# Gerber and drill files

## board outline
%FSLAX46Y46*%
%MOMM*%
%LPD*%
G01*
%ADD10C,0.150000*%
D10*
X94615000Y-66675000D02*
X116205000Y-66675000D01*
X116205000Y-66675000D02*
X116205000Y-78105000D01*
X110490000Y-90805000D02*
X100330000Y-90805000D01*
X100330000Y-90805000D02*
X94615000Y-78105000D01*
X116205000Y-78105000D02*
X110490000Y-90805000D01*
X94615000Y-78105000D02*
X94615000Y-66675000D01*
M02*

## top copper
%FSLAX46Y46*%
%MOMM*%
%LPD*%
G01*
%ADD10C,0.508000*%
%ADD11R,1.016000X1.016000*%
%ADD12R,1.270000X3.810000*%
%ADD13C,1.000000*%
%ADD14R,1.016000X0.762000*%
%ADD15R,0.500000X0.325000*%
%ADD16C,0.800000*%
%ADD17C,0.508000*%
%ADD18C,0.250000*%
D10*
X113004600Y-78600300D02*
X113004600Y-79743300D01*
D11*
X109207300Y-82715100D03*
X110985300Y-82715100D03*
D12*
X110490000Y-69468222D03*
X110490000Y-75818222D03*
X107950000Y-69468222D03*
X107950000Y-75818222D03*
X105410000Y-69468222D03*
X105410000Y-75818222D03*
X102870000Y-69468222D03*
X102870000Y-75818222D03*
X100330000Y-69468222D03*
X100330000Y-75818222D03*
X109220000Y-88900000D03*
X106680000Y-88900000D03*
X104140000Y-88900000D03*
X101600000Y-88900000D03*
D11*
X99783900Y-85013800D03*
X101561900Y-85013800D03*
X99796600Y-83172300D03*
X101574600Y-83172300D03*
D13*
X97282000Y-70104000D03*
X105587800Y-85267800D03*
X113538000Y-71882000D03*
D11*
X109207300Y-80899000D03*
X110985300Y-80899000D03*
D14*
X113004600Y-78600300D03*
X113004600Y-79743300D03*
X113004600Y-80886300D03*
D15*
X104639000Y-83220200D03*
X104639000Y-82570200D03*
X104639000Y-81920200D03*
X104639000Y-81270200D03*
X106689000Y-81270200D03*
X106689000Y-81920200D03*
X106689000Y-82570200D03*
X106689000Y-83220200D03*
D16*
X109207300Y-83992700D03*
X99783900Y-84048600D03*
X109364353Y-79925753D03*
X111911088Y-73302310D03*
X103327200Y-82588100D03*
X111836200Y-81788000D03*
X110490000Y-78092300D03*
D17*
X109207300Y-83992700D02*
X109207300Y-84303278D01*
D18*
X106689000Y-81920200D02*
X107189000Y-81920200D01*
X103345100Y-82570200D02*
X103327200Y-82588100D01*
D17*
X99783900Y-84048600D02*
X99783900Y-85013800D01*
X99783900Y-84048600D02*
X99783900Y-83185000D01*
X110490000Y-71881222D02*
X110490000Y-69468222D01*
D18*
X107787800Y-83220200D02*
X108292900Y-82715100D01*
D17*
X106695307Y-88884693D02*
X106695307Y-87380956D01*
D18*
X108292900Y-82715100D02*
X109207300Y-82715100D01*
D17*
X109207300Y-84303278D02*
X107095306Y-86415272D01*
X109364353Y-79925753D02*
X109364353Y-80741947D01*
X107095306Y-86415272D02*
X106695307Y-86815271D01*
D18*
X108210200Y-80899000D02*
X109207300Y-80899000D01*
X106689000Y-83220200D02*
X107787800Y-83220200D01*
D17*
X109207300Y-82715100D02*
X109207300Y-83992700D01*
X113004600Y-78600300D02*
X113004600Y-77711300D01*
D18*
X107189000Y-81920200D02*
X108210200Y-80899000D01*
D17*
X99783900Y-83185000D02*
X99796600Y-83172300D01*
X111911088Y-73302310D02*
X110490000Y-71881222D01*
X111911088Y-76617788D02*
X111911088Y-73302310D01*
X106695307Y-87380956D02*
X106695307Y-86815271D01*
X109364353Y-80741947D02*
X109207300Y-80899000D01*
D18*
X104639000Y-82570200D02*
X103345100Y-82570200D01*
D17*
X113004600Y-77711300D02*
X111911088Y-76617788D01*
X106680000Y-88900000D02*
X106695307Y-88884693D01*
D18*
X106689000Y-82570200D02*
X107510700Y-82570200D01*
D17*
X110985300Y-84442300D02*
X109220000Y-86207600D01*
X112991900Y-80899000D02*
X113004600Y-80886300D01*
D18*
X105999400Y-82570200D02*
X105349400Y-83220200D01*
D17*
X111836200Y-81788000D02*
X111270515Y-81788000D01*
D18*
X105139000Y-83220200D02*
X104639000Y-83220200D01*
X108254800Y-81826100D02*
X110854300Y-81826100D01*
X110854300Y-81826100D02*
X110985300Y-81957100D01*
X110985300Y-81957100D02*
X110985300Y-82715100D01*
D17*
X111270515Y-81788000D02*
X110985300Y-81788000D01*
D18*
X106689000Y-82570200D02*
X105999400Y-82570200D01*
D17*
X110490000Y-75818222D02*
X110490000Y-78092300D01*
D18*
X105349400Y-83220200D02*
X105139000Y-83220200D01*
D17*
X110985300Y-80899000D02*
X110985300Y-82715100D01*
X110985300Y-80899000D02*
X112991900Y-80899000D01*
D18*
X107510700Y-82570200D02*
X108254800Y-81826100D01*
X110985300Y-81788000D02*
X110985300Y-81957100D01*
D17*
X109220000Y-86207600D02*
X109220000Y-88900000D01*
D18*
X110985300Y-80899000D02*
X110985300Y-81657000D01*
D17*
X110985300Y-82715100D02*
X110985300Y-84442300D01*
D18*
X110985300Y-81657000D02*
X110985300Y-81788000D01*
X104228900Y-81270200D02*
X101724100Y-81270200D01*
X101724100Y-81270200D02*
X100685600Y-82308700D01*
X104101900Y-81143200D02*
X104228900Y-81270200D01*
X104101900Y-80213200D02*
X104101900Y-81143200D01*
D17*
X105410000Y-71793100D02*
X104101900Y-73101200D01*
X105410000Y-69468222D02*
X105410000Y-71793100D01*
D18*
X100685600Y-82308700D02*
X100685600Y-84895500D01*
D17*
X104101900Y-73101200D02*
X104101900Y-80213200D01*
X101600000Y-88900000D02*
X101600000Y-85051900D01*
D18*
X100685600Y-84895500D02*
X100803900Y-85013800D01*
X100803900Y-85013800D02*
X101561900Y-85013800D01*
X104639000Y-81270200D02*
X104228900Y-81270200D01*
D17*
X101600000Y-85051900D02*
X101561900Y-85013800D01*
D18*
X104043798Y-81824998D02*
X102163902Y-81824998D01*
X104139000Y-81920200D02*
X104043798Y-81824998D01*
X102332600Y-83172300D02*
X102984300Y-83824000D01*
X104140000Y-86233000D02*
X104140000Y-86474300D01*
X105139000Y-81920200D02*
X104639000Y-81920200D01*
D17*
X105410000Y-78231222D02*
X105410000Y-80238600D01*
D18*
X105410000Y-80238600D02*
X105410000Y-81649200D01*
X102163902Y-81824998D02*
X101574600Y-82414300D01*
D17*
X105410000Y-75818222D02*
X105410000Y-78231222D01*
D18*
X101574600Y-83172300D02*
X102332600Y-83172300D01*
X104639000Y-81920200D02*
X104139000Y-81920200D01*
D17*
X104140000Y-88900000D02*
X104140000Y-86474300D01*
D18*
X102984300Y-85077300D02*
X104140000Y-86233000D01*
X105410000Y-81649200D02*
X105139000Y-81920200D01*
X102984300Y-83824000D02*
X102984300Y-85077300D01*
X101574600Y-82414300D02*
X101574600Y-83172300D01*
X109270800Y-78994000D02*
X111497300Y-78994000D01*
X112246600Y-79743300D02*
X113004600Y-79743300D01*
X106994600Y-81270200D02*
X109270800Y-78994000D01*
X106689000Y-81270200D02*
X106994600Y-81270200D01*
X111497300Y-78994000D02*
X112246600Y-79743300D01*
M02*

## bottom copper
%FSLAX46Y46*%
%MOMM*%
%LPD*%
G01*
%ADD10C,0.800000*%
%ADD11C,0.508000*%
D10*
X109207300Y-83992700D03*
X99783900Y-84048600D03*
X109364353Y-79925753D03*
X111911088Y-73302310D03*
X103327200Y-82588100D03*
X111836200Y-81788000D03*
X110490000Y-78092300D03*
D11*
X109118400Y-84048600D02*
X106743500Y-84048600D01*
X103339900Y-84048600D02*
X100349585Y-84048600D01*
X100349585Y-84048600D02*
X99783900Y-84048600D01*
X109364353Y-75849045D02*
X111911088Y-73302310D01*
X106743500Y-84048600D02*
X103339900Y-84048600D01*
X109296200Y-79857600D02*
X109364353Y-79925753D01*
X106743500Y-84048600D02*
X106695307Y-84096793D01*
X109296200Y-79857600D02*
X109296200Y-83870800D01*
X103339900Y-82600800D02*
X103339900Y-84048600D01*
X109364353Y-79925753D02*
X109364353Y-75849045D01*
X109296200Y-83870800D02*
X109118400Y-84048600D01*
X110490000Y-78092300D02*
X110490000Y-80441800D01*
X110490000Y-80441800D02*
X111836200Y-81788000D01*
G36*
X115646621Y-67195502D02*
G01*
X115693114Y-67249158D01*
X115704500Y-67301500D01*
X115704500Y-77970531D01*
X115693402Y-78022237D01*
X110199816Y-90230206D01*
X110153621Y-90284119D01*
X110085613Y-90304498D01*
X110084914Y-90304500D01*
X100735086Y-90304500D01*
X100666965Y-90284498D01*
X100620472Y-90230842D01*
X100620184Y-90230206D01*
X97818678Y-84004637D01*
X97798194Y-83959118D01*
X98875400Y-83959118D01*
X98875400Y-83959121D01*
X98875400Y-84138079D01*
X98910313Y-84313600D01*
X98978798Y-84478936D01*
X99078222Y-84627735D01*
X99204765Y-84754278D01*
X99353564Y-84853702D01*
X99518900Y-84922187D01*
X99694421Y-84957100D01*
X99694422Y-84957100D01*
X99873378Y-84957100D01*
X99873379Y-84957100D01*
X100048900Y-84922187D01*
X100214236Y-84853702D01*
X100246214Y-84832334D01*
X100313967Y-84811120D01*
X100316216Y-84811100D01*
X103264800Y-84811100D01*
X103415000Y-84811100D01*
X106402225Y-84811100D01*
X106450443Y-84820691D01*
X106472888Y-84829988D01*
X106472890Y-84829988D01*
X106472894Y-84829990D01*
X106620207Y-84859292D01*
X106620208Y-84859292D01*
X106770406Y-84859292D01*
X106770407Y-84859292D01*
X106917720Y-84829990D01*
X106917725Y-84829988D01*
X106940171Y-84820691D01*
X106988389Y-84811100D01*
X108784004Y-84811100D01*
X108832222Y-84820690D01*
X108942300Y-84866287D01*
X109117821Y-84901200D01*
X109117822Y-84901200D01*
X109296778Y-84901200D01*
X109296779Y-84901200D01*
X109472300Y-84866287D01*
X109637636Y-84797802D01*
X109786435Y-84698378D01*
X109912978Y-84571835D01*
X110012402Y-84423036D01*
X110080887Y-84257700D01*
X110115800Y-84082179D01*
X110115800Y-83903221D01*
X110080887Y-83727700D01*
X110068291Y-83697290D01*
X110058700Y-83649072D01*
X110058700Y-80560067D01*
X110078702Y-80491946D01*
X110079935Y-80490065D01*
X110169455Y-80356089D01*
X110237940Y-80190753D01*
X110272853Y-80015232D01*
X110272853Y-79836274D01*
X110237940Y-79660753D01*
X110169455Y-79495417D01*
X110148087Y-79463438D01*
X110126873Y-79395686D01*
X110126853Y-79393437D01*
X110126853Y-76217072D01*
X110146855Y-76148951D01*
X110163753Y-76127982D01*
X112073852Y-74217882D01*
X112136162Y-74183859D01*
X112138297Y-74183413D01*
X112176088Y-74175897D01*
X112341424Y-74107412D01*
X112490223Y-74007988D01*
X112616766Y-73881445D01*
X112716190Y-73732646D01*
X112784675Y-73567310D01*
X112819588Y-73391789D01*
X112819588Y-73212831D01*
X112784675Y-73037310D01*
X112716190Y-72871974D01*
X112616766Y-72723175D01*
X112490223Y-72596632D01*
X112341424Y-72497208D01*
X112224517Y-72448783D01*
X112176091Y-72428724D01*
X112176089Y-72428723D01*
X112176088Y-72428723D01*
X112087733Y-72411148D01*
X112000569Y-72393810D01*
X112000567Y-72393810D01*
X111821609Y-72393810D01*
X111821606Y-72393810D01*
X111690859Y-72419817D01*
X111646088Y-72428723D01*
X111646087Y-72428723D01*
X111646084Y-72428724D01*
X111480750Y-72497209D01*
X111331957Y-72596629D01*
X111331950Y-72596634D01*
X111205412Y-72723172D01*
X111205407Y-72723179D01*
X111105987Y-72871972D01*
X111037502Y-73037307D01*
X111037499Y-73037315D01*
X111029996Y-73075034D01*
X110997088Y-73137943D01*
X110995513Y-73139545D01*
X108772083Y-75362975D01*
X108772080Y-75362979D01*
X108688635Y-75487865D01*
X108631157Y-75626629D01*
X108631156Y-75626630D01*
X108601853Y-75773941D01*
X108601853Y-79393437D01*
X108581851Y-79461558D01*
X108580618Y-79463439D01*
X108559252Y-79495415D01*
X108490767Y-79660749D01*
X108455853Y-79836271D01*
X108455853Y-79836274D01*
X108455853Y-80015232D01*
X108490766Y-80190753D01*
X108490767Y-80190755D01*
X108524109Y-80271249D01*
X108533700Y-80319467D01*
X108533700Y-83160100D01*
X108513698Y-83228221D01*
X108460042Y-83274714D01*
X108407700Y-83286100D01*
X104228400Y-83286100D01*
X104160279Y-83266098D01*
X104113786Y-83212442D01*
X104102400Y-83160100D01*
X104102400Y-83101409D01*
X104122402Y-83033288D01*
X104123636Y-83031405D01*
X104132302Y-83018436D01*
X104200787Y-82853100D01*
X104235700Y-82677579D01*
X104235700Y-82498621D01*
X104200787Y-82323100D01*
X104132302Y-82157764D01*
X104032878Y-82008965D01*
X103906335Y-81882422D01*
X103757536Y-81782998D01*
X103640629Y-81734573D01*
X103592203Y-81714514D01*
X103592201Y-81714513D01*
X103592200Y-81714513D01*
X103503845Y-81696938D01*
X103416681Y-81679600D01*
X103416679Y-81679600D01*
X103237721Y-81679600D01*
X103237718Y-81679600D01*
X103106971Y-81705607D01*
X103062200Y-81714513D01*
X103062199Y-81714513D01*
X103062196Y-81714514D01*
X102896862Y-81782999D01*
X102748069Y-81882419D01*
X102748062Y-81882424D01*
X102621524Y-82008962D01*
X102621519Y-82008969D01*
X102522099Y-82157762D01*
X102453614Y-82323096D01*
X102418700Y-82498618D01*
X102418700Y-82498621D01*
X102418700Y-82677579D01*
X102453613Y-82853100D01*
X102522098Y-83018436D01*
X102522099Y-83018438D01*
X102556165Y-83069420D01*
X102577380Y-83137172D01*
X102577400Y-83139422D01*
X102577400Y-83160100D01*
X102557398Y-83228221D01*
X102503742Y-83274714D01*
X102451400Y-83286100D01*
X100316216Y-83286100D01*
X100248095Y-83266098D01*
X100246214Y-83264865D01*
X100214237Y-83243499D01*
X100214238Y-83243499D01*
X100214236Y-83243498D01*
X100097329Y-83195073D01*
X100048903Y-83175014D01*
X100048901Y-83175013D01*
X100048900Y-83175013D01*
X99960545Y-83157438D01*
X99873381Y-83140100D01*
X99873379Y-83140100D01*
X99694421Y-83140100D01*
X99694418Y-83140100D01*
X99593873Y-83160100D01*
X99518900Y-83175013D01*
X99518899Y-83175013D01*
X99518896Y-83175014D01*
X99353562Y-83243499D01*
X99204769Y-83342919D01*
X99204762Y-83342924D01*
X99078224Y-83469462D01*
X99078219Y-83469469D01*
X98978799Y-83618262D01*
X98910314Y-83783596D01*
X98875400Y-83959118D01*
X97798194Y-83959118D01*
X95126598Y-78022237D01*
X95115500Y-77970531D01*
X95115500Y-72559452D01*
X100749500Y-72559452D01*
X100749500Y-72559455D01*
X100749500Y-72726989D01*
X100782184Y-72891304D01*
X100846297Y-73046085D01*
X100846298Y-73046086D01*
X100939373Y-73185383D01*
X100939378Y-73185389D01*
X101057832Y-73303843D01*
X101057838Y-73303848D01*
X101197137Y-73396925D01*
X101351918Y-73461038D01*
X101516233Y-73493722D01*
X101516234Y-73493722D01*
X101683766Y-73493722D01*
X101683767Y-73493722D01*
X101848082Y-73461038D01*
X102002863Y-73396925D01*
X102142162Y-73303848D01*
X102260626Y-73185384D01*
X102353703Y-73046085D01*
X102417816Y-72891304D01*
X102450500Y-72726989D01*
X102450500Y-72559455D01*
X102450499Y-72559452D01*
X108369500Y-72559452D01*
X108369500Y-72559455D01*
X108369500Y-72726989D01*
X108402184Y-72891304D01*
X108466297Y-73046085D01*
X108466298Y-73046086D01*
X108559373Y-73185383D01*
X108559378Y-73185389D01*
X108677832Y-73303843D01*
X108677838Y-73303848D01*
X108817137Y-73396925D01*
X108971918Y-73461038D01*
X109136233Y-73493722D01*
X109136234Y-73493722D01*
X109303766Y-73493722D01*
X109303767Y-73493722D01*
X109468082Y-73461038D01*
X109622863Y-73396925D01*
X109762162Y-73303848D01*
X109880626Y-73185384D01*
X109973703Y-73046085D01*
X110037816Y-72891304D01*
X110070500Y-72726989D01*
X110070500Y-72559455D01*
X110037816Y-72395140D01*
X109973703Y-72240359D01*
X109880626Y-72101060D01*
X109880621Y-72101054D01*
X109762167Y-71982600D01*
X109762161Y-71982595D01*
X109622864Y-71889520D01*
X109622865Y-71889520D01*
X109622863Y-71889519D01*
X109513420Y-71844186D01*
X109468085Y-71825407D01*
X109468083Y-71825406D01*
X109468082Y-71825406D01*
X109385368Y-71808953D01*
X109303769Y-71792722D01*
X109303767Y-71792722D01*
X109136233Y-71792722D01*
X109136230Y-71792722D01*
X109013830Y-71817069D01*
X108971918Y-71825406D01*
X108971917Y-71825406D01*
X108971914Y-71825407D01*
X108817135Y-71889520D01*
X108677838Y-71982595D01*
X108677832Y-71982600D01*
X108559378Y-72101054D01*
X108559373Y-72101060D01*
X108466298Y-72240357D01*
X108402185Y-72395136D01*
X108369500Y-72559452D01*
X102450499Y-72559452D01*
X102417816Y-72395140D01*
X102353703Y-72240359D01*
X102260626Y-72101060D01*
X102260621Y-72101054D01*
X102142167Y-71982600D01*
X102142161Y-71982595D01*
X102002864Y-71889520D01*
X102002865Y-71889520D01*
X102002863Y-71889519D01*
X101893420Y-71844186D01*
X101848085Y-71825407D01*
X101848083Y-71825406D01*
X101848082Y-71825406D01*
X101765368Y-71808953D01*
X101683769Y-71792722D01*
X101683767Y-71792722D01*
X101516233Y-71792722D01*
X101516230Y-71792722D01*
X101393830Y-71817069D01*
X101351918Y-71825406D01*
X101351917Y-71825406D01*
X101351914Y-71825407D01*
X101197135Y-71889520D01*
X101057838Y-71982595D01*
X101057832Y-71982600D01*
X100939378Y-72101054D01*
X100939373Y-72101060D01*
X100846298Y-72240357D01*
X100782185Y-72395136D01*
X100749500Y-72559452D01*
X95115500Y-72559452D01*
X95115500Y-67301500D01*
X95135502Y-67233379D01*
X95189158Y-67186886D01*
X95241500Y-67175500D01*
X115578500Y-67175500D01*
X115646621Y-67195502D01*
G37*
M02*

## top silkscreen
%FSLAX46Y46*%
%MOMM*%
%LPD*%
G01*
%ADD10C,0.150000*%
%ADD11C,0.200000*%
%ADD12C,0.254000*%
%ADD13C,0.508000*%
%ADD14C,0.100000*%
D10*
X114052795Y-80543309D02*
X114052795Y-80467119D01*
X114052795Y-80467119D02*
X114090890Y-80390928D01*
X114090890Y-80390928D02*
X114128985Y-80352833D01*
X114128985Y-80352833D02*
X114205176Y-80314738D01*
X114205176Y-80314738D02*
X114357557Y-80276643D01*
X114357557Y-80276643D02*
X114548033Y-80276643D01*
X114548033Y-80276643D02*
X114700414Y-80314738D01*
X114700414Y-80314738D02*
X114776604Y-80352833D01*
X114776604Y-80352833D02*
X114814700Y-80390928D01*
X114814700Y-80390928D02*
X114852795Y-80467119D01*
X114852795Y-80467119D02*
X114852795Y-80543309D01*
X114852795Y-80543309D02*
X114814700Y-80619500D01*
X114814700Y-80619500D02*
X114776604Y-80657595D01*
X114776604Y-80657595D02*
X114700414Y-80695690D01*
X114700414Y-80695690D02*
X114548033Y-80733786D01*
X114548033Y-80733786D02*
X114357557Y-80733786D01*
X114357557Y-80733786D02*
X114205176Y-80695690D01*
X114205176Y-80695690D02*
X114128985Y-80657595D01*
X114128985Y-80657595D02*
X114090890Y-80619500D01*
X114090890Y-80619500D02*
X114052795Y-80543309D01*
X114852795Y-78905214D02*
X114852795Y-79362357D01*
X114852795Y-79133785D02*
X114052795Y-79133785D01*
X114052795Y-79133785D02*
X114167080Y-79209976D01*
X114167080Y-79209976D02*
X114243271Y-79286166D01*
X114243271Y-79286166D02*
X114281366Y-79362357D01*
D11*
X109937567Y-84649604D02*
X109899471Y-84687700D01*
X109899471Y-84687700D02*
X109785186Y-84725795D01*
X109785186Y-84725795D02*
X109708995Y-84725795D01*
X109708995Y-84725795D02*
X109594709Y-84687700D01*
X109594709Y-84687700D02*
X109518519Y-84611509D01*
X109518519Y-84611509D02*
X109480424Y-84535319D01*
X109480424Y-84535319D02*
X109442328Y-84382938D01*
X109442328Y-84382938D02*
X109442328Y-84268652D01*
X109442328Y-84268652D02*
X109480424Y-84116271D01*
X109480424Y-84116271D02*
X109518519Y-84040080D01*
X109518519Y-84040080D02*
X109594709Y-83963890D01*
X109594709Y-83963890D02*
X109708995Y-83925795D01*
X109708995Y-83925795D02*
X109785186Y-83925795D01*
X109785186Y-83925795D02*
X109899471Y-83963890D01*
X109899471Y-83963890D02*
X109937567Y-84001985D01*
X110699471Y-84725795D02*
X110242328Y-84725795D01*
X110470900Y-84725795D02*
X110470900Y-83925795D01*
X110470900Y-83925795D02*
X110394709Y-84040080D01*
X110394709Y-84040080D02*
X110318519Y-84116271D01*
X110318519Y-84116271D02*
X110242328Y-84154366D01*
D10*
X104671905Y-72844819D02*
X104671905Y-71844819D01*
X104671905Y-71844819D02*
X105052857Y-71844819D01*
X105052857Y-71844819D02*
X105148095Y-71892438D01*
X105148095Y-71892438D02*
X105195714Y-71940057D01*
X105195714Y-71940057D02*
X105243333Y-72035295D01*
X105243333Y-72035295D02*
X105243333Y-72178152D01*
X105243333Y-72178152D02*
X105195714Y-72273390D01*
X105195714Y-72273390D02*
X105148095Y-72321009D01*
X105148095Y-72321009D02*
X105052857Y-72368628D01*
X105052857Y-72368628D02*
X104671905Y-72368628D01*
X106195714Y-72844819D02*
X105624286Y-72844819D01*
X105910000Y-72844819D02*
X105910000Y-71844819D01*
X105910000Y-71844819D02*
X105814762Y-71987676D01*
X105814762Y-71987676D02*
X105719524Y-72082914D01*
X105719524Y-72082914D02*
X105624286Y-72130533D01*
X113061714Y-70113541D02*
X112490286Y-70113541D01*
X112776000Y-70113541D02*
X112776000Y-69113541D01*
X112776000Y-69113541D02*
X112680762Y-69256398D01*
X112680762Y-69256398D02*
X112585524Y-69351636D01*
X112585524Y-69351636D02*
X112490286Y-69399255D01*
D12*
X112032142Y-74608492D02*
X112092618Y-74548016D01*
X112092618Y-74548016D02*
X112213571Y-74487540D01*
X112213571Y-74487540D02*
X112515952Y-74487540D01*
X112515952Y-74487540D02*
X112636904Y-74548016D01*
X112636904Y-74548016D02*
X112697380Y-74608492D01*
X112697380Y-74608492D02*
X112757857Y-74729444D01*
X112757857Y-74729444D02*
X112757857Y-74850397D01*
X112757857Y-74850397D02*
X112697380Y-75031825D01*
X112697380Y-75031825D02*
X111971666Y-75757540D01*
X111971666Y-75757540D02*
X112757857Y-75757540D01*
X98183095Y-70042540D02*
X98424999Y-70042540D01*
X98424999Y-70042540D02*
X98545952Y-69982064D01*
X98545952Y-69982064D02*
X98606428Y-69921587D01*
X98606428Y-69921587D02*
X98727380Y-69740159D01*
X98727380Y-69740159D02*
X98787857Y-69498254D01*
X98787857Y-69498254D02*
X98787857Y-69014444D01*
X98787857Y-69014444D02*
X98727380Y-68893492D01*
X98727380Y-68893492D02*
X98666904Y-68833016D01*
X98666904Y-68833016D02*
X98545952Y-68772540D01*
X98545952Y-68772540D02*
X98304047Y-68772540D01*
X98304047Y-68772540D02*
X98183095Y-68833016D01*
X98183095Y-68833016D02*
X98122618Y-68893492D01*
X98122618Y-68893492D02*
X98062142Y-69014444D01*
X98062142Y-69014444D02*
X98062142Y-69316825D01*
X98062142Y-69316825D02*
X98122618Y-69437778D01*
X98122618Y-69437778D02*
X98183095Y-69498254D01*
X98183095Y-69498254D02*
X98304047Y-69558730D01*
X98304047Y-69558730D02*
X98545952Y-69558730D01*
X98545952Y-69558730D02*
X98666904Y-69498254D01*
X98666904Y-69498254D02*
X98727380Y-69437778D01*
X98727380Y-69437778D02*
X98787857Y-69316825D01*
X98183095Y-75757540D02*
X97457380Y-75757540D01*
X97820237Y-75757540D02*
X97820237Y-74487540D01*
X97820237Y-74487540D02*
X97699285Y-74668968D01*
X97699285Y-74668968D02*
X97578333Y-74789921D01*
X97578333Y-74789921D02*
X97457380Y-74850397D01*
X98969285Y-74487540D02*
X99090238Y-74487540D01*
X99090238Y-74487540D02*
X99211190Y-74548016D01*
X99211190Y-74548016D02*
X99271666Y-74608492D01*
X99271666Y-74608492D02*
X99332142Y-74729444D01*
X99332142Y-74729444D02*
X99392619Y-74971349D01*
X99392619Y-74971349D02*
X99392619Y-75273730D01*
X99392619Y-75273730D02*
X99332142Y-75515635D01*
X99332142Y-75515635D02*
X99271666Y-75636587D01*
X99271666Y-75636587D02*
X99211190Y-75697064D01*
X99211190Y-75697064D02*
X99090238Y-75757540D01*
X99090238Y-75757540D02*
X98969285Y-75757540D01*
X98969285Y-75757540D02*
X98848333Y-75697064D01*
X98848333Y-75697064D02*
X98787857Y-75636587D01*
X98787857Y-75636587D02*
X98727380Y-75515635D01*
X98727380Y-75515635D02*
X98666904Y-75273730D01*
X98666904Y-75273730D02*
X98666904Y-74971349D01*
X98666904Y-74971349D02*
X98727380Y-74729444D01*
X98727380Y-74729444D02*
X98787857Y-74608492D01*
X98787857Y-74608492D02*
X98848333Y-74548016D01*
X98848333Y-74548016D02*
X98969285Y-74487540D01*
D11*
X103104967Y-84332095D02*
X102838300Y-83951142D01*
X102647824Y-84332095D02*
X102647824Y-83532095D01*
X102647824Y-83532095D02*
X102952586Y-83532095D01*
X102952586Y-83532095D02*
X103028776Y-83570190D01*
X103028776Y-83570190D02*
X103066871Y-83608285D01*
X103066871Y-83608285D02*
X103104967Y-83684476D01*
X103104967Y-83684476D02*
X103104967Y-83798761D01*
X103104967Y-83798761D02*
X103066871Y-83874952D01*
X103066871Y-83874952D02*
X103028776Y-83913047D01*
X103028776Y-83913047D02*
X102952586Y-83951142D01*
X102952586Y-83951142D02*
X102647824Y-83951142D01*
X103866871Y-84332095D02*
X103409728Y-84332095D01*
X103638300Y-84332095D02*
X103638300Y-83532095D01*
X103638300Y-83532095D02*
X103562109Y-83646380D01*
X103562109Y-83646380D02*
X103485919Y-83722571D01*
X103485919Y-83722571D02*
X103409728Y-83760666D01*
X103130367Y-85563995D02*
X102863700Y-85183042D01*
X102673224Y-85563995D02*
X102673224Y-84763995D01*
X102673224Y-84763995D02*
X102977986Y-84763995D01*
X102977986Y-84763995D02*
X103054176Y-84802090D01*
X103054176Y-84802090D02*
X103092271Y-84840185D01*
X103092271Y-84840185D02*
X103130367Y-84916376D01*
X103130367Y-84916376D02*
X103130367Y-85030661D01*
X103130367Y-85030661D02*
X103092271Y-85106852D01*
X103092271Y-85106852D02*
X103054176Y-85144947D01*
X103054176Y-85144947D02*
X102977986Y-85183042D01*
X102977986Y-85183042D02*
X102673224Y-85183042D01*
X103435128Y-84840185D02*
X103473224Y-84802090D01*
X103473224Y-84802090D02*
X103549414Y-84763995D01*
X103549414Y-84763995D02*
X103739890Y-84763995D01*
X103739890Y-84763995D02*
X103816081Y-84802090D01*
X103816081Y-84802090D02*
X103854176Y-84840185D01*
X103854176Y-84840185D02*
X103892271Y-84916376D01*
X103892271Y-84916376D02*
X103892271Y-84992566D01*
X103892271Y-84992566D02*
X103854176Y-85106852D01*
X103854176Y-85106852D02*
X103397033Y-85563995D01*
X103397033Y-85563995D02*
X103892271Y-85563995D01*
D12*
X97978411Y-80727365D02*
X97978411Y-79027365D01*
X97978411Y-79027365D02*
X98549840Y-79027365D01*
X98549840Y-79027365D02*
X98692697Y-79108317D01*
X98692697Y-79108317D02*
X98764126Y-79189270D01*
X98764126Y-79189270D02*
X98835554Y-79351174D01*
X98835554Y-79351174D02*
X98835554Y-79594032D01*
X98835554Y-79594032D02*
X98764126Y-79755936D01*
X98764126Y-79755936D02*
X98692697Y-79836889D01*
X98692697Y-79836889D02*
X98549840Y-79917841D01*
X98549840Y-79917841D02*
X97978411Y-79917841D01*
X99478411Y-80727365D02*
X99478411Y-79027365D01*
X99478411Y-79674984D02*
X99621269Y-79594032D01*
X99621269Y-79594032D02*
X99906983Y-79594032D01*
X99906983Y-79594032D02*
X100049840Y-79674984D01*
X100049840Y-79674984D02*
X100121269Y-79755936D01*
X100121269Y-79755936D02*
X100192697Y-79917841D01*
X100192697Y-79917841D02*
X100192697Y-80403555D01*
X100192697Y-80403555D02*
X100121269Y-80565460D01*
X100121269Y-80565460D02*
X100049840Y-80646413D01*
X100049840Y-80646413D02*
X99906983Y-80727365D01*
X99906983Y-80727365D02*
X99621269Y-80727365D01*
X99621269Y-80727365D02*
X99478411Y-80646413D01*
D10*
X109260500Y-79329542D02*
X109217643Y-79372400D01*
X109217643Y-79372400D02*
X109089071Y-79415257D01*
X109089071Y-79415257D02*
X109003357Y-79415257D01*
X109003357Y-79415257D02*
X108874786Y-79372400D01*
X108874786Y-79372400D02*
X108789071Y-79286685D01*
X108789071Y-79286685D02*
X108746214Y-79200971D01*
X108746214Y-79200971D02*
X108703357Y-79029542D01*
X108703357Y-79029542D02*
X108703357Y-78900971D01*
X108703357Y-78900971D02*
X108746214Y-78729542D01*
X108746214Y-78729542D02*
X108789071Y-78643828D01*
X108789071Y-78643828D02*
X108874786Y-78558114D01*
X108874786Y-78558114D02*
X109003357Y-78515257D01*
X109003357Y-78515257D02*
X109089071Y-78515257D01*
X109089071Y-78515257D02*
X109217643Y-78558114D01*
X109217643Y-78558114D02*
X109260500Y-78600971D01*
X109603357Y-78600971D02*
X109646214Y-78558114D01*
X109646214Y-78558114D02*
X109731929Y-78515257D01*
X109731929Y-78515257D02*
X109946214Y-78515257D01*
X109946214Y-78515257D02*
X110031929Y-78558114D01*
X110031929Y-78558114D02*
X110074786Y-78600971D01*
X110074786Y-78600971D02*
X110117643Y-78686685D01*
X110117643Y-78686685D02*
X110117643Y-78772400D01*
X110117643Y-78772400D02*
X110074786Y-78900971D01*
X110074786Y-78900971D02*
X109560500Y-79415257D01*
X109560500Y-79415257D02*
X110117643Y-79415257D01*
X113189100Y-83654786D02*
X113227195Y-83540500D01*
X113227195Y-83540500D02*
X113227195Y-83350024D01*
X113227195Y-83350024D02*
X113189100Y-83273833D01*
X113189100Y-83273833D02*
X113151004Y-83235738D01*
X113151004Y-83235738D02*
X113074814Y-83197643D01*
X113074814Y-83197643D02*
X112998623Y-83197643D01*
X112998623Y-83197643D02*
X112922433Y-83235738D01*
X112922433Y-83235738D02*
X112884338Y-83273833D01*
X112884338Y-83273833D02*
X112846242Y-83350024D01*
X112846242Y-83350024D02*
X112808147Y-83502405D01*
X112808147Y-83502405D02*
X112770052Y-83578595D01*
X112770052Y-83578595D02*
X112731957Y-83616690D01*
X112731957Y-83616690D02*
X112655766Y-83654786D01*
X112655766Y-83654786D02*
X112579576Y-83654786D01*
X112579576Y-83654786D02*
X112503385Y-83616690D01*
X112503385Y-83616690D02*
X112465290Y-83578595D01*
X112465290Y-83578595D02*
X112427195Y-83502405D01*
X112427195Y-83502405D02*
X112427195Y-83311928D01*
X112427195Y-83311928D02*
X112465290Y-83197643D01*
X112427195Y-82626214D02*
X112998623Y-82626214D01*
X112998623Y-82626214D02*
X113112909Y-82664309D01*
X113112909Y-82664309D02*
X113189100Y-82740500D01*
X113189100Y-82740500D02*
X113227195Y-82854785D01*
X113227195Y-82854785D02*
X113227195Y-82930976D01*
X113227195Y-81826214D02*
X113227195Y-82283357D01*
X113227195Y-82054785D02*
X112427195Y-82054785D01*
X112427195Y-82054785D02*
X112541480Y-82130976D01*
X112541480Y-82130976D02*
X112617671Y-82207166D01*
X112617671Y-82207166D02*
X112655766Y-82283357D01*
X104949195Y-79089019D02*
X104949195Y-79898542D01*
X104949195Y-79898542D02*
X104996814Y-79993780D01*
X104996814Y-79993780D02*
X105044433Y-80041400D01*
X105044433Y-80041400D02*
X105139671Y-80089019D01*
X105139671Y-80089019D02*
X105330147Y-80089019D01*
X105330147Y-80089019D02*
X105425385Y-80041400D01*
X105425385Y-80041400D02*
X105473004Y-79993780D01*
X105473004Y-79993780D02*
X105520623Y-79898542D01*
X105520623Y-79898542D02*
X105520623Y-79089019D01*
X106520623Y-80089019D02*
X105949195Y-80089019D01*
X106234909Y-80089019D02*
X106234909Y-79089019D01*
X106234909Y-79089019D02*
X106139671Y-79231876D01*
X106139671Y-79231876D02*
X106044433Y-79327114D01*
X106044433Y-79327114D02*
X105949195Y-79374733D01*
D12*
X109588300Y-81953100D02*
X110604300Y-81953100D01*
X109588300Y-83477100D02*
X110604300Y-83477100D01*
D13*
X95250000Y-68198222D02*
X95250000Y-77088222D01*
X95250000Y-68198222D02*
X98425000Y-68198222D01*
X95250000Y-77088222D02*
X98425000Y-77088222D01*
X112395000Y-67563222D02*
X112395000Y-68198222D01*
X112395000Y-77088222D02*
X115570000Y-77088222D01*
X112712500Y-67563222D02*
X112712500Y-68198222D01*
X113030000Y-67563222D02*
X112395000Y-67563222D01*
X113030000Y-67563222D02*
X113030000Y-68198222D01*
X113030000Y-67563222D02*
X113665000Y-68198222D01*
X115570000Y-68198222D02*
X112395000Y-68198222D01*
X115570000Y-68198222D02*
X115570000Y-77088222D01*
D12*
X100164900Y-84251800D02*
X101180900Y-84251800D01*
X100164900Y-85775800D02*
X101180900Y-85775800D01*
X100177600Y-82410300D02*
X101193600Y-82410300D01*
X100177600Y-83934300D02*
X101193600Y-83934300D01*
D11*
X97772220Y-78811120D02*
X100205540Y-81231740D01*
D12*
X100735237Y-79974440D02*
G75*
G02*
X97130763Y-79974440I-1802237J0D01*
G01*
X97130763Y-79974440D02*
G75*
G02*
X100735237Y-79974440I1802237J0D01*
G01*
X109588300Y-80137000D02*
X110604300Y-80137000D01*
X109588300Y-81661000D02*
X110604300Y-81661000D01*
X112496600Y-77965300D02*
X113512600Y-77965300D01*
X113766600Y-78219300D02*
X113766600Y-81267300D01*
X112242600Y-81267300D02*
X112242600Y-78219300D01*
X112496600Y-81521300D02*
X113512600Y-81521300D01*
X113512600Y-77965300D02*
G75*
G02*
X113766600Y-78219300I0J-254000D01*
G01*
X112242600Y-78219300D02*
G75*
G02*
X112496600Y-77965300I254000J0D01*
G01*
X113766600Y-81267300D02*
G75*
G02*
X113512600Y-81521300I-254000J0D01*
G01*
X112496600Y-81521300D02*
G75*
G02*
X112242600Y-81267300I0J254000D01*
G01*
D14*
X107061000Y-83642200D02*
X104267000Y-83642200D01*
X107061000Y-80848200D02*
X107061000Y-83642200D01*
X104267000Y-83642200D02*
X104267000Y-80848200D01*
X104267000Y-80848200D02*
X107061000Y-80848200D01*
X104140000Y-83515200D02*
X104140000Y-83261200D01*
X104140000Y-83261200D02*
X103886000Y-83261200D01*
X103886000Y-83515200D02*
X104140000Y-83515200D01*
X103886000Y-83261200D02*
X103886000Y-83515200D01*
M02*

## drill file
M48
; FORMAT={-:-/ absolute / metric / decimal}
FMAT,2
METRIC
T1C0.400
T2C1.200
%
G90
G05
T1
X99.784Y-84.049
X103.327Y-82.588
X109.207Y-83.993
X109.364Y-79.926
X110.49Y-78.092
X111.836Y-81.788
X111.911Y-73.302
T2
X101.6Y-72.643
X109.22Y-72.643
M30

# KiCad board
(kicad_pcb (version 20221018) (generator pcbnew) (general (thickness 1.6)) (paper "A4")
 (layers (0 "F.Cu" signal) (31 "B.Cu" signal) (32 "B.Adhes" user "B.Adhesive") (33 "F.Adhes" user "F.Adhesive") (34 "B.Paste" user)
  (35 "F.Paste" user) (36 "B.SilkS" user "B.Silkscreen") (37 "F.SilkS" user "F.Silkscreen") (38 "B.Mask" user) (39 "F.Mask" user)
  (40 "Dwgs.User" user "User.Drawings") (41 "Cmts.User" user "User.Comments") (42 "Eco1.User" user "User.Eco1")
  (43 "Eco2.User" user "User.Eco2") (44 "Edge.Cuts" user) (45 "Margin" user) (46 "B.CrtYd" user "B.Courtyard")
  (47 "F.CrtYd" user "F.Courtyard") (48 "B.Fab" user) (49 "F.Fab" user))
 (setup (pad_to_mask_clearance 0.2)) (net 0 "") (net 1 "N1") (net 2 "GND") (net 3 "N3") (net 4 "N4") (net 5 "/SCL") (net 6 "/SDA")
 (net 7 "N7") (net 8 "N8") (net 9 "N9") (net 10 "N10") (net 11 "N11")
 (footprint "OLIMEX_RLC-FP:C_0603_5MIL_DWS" (layer "F.Cu") (at 110.0963 82.7151)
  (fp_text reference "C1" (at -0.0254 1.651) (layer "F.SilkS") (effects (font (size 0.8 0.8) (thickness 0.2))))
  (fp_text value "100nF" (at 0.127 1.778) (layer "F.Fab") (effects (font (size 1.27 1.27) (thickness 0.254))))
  (fp_line (start -0.508 -0.762) (end 0.508 -0.762) (stroke (width 0.254) (type solid)) (layer "F.SilkS"))
  (fp_line (start -0.508 0.762) (end 0.508 0.762) (stroke (width 0.254) (type solid)) (layer "F.SilkS"))
  (pad "1" smd rect (at -0.889 0) (size 1.016 1.016) (layers "F.Cu" "F.Paste" "F.Mask") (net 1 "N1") (solder_mask_margin 0.0508)
   (clearance 0.0508))
  (pad "2" smd rect (at 0.889 0) (size 1.016 1.016) (layers "F.Cu" "F.Paste" "F.Mask") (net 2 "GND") (solder_mask_margin 0.0508)
   (clearance 0.0508)))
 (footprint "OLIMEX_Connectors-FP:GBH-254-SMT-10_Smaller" (layer "F.Cu") (at 105.41 72.643222) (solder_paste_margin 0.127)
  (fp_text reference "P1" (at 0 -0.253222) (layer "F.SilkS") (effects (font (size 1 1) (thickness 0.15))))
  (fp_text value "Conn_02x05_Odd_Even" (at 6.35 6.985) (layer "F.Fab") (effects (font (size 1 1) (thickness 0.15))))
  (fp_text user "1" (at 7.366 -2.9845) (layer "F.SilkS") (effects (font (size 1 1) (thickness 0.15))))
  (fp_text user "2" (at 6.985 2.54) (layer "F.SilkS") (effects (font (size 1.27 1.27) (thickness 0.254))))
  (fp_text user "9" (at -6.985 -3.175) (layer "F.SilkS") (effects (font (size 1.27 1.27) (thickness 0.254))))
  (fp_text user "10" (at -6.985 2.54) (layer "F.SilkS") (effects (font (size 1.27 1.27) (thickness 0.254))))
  (fp_line (start -10.16 -4.445) (end -10.16 4.445) (stroke (width 0.508) (type solid)) (layer "F.SilkS"))
  (fp_line (start -10.16 -4.445) (end -6.985 -4.445) (stroke (width 0.508) (type solid)) (layer "F.SilkS"))
  (fp_line (start -10.16 4.445) (end -6.985 4.445) (stroke (width 0.508) (type solid)) (layer "F.SilkS"))
  (fp_line (start 6.985 -5.08) (end 6.985 -4.445) (stroke (width 0.508) (type solid)) (layer "F.SilkS"))
  (fp_line (start 6.985 4.445) (end 10.16 4.445) (stroke (width 0.508) (type solid)) (layer "F.SilkS"))
  (fp_line (start 7.3025 -5.08) (end 7.3025 -4.445) (stroke (width 0.508) (type solid)) (layer "F.SilkS"))
  (fp_line (start 7.62 -5.08) (end 6.985 -5.08) (stroke (width 0.508) (type solid)) (layer "F.SilkS"))
  (fp_line (start 7.62 -5.08) (end 7.62 -4.445) (stroke (width 0.508) (type solid)) (layer "F.SilkS"))
  (fp_line (start 7.62 -5.08) (end 8.255 -4.445) (stroke (width 0.508) (type solid)) (layer "F.SilkS"))
  (fp_line (start 10.16 -4.445) (end 6.985 -4.445) (stroke (width 0.508) (type solid)) (layer "F.SilkS"))
  (fp_line (start 10.16 -4.445) (end 10.16 4.445) (stroke (width 0.508) (type solid)) (layer "F.SilkS"))
  (pad "" smd trapezoid (at -5.08 -3.175) (size 1.7 3.81) (layers "F.Paste"))
  (pad "" smd trapezoid (at -5.08 3.175) (size 1.7 3.81) (layers "F.Paste"))
  (pad "" np_thru_hole circle (at -3.81 0) (size 1.2 1.2) (drill 1.2) (layers "*.Cu" "*.Mask") (solder_mask_margin 0.0508))
  (pad "" smd trapezoid (at -2.54 -3.175) (size 1.7 3.81) (layers "F.Paste"))
  (pad "" smd trapezoid (at -2.54 3.175) (size 1.7 3.81) (layers "F.Paste"))
  (pad "" smd trapezoid (at 0 -3.175) (size 1.7 3.81) (layers "F.Paste"))
  (pad "" smd trapezoid (at 0 3.175) (size 1.7 3.81) (layers "F.Paste"))
  (pad "" smd trapezoid (at 2.54 -3.175) (size 1.7 3.81) (layers "F.Paste"))
  (pad "" smd trapezoid (at 2.54 3.175) (size 1.7 3.81) (layers "F.Paste"))
  (pad "" np_thru_hole circle (at 3.81 0) (size 1.2 1.2) (drill 1.2) (layers "*.Cu" "*.Mask") (solder_mask_margin 0.0508))
  (pad "" smd trapezoid (at 5.08 -3.175) (size 1.7 3.81) (layers "F.Paste"))
  (pad "" smd trapezoid (at 5.08 3.175) (size 1.7 3.81) (layers "F.Paste"))
  (pad "1" smd rect (at 5.08 -3.175) (size 1.27 3.81) (layers "F.Cu" "F.Mask") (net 1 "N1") (solder_mask_margin 0.0508)
   (solder_paste_margin 0.127) (clearance 0.0508))
  (pad "2" smd rect (at 5.08 3.175) (size 1.27 3.81) (layers "F.Cu" "F.Mask") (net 2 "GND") (solder_mask_margin 0.0508)
   (solder_paste_margin 0.127) (clearance 0.0508))
  (pad "3" smd rect (at 2.54 -3.175) (size 1.27 3.81) (layers "F.Cu" "F.Mask") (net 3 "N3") (solder_mask_margin 0.0508)
   (solder_paste_margin 0.127) (clearance 0.0508))
  (pad "4" smd rect (at 2.54 3.175) (size 1.27 3.81) (layers "F.Cu" "F.Mask") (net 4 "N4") (solder_mask_margin 0.0508)
   (solder_paste_margin 0.127) (clearance 0.0508))
  (pad "5" smd rect (at 0 -3.175) (size 1.27 3.81) (layers "F.Cu" "F.Mask") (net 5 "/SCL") (solder_mask_margin 0.0508)
   (solder_paste_margin 0.127) (clearance 0.0508))
  (pad "6" smd rect (at 0 3.175) (size 1.27 3.81) (layers "F.Cu" "F.Mask") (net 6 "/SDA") (solder_mask_margin 0.0508)
   (solder_paste_margin 0.127) (clearance 0.0508))
  (pad "7" smd rect (at -2.54 -3.175) (size 1.27 3.81) (layers "F.Cu" "F.Mask") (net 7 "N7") (solder_mask_margin 0.0508)
   (solder_paste_margin 0.127) (clearance 0.0508))
  (pad "8" smd rect (at -2.54 3.175) (size 1.27 3.81) (layers "F.Cu" "F.Mask") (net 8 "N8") (solder_mask_margin 0.0508)
   (solder_paste_margin 0.127) (clearance 0.0508))
  (pad "9" smd rect (at -5.08 -3.175) (size 1.27 3.81) (layers "F.Cu" "F.Mask") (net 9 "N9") (solder_mask_margin 0.0508)
   (solder_paste_margin 0.127) (clearance 0.0508))
  (pad "10" smd rect (at -5.08 3.175) (size 1.27 3.81) (layers "F.Cu" "F.Mask") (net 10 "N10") (solder_mask_margin 0.0508)
   (solder_paste_margin 0.127) (clearance 0.0508)))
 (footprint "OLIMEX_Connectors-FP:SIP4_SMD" (layer "F.Cu") (at 105.41 88.9 180)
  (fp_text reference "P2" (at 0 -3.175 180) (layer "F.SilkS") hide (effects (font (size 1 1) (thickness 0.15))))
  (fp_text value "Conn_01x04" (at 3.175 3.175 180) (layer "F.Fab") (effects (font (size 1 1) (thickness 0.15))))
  (pad "1" smd rect (at -3.81 0 180) (size 1.27 3.81) (layers "F.Cu" "F.Mask") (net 2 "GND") (solder_mask_margin 0.0508)
   (solder_paste_margin -0.0508) (clearance 0.0508))
  (pad "2" smd rect (at -1.27 0 180) (size 1.27 3.81) (layers "F.Cu" "F.Mask") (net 1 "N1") (solder_mask_margin 0.0508)
   (solder_paste_margin -0.0508) (clearance 0.0508))
  (pad "3" smd rect (at 1.27 0 180) (size 1.27 3.81) (layers "F.Cu" "F.Mask") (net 6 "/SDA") (solder_mask_margin 0.0508)
   (solder_paste_margin -0.0508) (clearance 0.0508))
  (pad "4" smd rect (at 3.81 0 180) (size 1.27 3.81) (layers "F.Cu" "F.Mask") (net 5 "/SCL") (solder_mask_margin 0.0508)
   (solder_paste_margin -0.0508) (clearance 0.0508)))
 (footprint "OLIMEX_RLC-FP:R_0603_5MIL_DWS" (layer "F.Cu") (at 100.6729 85.0138)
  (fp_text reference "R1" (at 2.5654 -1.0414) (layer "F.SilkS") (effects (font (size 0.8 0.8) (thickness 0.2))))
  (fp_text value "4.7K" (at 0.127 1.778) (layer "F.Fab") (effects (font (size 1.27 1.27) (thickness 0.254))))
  (fp_line (start -0.508 -0.762) (end 0.508 -0.762) (stroke (width 0.254) (type solid)) (layer "F.SilkS"))
  (fp_line (start -0.508 0.762) (end 0.508 0.762) (stroke (width 0.254) (type solid)) (layer "F.SilkS"))
  (pad "1" smd rect (at -0.889 0) (size 1.016 1.016) (layers "F.Cu" "F.Paste" "F.Mask") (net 1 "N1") (solder_mask_margin 0.0508))
  (pad "2" smd rect (at 0.889 0) (size 1.016 1.016) (layers "F.Cu" "F.Paste" "F.Mask") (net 5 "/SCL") (solder_mask_margin 0.0508)))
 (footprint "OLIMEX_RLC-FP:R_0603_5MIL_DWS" (layer "F.Cu") (at 100.6856 83.1723)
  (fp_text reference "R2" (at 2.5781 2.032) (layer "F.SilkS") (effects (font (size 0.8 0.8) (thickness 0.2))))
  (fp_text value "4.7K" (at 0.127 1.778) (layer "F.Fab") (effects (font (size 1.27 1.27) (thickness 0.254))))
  (fp_line (start -0.508 -0.762) (end 0.508 -0.762) (stroke (width 0.254) (type solid)) (layer "F.SilkS"))
  (fp_line (start -0.508 0.762) (end 0.508 0.762) (stroke (width 0.254) (type solid)) (layer "F.SilkS"))
  (pad "1" smd rect (at -0.889 0) (size 1.016 1.016) (layers "F.Cu" "F.Paste" "F.Mask") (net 1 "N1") (solder_mask_margin 0.0508))
  (pad "2" smd rect (at 0.889 0) (size 1.016 1.016) (layers "F.Cu" "F.Paste" "F.Mask") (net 6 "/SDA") (solder_mask_margin 0.0508)))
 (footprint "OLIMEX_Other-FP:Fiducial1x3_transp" (layer "F.Cu") (at 97.282 70.104)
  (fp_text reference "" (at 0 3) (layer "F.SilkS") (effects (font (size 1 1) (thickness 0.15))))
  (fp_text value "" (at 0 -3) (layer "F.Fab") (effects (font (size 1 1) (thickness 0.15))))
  (pad "Fid1" connect circle (at 0 0) (size 1 1) (layers "F.Cu" "F.Mask") (solder_mask_margin 0.127) (clearance 1.016) (zone_connect 0)))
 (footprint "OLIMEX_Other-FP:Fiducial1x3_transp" (layer "F.Cu") (at 105.5878 85.2678)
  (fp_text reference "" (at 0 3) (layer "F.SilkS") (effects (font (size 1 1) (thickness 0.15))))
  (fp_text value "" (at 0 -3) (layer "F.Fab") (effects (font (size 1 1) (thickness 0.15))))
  (pad "Fid1" connect circle (at 0 0) (size 1 1) (layers "F.Cu" "F.Mask") (solder_mask_margin 0.127) (clearance 1.016) (zone_connect 0)))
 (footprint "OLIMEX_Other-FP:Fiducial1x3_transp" (layer "F.Cu") (at 113.538 71.882)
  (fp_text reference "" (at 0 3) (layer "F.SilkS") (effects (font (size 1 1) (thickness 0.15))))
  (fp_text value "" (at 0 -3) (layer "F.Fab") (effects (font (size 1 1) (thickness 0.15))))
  (pad "Fid1" connect circle (at 0 0) (size 1 1) (layers "F.Cu" "F.Mask") (solder_mask_margin 0.127) (clearance 1.016) (zone_connect 0)))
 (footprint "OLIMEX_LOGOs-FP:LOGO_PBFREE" (layer "F.Cu") (at 99.1362 80.2894)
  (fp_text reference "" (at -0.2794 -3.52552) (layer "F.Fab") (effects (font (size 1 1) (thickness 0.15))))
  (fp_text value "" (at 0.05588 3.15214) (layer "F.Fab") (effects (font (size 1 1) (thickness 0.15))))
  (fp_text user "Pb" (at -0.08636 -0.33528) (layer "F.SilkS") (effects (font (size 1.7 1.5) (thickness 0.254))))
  (fp_line (start -1.36398 -1.47828) (end 1.06934 0.94234) (stroke (width 0.2) (type solid)) (layer "F.SilkS"))
  (fp_circle (center -0.2032 -0.31496) (end 0.90678 -1.73482) (stroke (width 0.254) (type solid)) (fill none) (layer "F.SilkS")))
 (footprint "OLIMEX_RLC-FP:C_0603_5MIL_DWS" (layer "F.Cu") (at 110.0963 80.899)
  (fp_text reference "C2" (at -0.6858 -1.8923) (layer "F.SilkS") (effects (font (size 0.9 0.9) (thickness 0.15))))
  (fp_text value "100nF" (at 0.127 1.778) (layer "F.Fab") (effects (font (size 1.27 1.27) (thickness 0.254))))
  (fp_line (start -0.508 -0.762) (end 0.508 -0.762) (stroke (width 0.254) (type solid)) (layer "F.SilkS"))
  (fp_line (start -0.508 0.762) (end 0.508 0.762) (stroke (width 0.254) (type solid)) (layer "F.SilkS"))
  (pad "1" smd rect (at -0.889 0) (size 1.016 1.016) (layers "F.Cu" "F.Paste" "F.Mask") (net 1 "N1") (solder_mask_margin 0.0508)
   (clearance 0.0508))
  (pad "2" smd rect (at 0.889 0) (size 1.016 1.016) (layers "F.Cu" "F.Paste" "F.Mask") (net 2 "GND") (solder_mask_margin 0.0508)
   (clearance 0.0508)))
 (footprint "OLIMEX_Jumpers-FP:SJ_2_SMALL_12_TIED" (layer "F.Cu") (at 113.0046 79.7433 -90)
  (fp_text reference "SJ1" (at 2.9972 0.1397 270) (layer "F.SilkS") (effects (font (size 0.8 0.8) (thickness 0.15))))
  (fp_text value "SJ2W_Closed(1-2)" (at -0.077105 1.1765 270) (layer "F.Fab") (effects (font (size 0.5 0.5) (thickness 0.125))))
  (fp_line (start -1.143 0) (end 0 0) (stroke (width 0.508) (type solid)) (layer "F.Cu"))
  (fp_line (start -1.778 0.508) (end -1.778 -0.508) (stroke (width 0.254) (type solid)) (layer "F.SilkS"))
  (fp_line (start -1.524 -0.762) (end 1.524 -0.762) (stroke (width 0.254) (type solid)) (layer "F.SilkS"))
  (fp_line (start 1.524 0.762) (end -1.524 0.762) (stroke (width 0.254) (type solid)) (layer "F.SilkS"))
  (fp_line (start 1.778 0.508) (end 1.778 -0.508) (stroke (width 0.254) (type solid)) (layer "F.SilkS"))
  (fp_arc (start -1.778 -0.508) (mid -1.703605 -0.687605) (end -1.524 -0.762) (stroke (width 0.254) (type solid)) (layer "F.SilkS"))
  (fp_arc (start -1.524 0.762) (mid -1.703605 0.687605) (end -1.778 0.508) (stroke (width 0.254) (type solid)) (layer "F.SilkS"))
  (fp_arc (start 1.524 -0.762) (mid 1.703605 -0.687605) (end 1.778 -0.508) (stroke (width 0.254) (type solid)) (layer "F.SilkS"))
  (fp_arc (start 1.778 0.508) (mid 1.703605 0.687605) (end 1.524 0.762) (stroke (width 0.254) (type solid)) (layer "F.SilkS"))
  (pad "1" smd rect (at -1.143 0 270) (size 0.762 1.016) (layers "F.Cu" "F.Mask") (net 1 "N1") (solder_mask_margin 0.0508)
   (solder_paste_margin -0.0508) (clearance 0.0508))
  (pad "2" smd rect (at 0 0 270) (size 0.762 1.016) (layers "F.Cu" "F.Mask") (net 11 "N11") (solder_mask_margin 0.0508)
   (solder_paste_margin -0.0508) (clearance 0.0508))
  (pad "3" smd rect (at 1.143 0 270) (size 0.762 1.016) (layers "F.Cu" "F.Mask") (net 2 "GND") (solder_mask_margin 0.0508)
   (solder_paste_margin -0.0508) (clearance 0.0508)))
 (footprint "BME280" (layer "F.Cu") (at 105.664 82.2452 180)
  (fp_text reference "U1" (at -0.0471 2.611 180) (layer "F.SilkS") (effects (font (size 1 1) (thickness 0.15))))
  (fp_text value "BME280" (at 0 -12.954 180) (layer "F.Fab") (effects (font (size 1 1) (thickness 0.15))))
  (fp_line (start -1.397 -1.397) (end 1.397 -1.397) (stroke (width 0.1) (type solid)) (layer "F.SilkS"))
  (fp_line (start -1.397 1.397) (end -1.397 -1.397) (stroke (width 0.1) (type solid)) (layer "F.SilkS"))
  (fp_line (start 1.397 -1.397) (end 1.397 1.397) (stroke (width 0.1) (type solid)) (layer "F.SilkS"))
  (fp_line (start 1.397 1.397) (end -1.397 1.397) (stroke (width 0.1) (type solid)) (layer "F.SilkS"))
  (fp_line (start 1.524 -1.27) (end 1.524 -1.016) (stroke (width 0.1) (type solid)) (layer "F.SilkS"))
  (fp_line (start 1.524 -1.016) (end 1.778 -1.016) (stroke (width 0.1) (type solid)) (layer "F.SilkS"))
  (fp_line (start 1.778 -1.27) (end 1.524 -1.27) (stroke (width 0.1) (type solid)) (layer "F.SilkS"))
  (fp_line (start 1.778 -1.016) (end 1.778 -1.27) (stroke (width 0.1) (type solid)) (layer "F.SilkS"))
  (pad "1" smd rect (at 1.025 -0.975 180) (size 0.5 0.325) (layers "F.Cu" "F.Paste" "F.Mask") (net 2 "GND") (solder_mask_margin 0.05))
  (pad "2" smd rect (at 1.025 -0.325 180) (size 0.5 0.325) (layers "F.Cu" "F.Paste" "F.Mask") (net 1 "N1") (solder_mask_margin 0.05))
  (pad "3" smd rect (at 1.025 0.325 180) (size 0.5 0.325) (layers "F.Cu" "F.Paste" "F.Mask") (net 6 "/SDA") (solder_mask_margin 0.05))
  (pad "4" smd rect (at 1.025 0.975 180) (size 0.5 0.325) (layers "F.Cu" "F.Paste" "F.Mask") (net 5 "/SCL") (solder_mask_margin 0.05))
  (pad "5" smd rect (at -1.025 0.975 180) (size 0.5 0.325) (layers "F.Cu" "F.Paste" "F.Mask") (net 11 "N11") (solder_mask_margin 0.05))
  (pad "6" smd rect (at -1.025 0.325 180) (size 0.5 0.325) (layers "F.Cu" "F.Paste" "F.Mask") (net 1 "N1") (solder_mask_margin 0.05))
  (pad "7" smd rect (at -1.025 -0.325 180) (size 0.5 0.325) (layers "F.Cu" "F.Paste" "F.Mask") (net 2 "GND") (solder_mask_margin 0.05))
  (pad "8" smd rect (at -1.025 -0.975 180) (size 0.5 0.325) (layers "F.Cu" "F.Paste" "F.Mask") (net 1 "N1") (solder_mask_margin 0.05)))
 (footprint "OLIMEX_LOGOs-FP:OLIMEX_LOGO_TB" (layer "B.Cu") (at 105.41 69.85 180)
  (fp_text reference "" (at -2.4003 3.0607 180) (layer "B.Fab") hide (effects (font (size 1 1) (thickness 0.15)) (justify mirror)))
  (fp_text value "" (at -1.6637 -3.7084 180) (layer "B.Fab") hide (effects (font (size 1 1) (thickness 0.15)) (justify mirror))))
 (gr_line (start 94.615 66.675) (end 116.205 66.675) (stroke (width 0.15) (type solid)) (layer "Edge.Cuts"))
 (gr_line (start 116.205 66.675) (end 116.205 78.105) (stroke (width 0.15) (type solid)) (layer "Edge.Cuts"))
 (gr_line (start 110.49 90.805) (end 100.33 90.805) (stroke (width 0.15) (type solid)) (layer "Edge.Cuts"))
 (gr_line (start 100.33 90.805) (end 94.615 78.105) (stroke (width 0.15) (type solid)) (layer "Edge.Cuts"))
 (gr_line (start 116.205 78.105) (end 110.49 90.805) (stroke (width 0.15) (type solid)) (layer "Edge.Cuts"))
 (gr_line (start 94.615 78.105) (end 94.615 66.675) (stroke (width 0.15) (type solid)) (layer "Edge.Cuts"))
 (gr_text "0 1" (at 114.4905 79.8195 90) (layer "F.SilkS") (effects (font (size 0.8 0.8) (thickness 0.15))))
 (segment (start 109.2073 83.9927) (end 109.2073 84.303278) (width 0.508) (layer "F.Cu") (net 1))
 (segment (start 106.689 81.9202) (end 107.189 81.9202) (width 0.25) (layer "F.Cu") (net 1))
 (segment (start 103.3451 82.5702) (end 103.3272 82.5881) (width 0.25) (layer "F.Cu") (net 1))
 (segment (start 99.7839 84.0486) (end 99.7839 85.0138) (width 0.508) (layer "F.Cu") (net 1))
 (segment (start 99.7839 84.0486) (end 99.7839 83.185) (width 0.508) (layer "F.Cu") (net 1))
 (segment (start 110.49 71.881222) (end 110.49 69.468222) (width 0.508) (layer "F.Cu") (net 1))
 (segment (start 107.7878 83.2202) (end 108.2929 82.7151) (width 0.25) (layer "F.Cu") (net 1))
 (segment (start 106.695307 88.884693) (end 106.695307 87.380956) (width 0.508) (layer "F.Cu") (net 1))
 (segment (start 108.2929 82.7151) (end 109.2073 82.7151) (width 0.25) (layer "F.Cu") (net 1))
 (segment (start 109.2073 84.303278) (end 107.095306 86.415272) (width 0.508) (layer "F.Cu") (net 1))
 (segment (start 109.364353 79.925753) (end 109.364353 80.741947) (width 0.508) (layer "F.Cu") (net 1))
 (segment (start 107.095306 86.415272) (end 106.695307 86.815271) (width 0.508) (layer "F.Cu") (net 1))
 (segment (start 108.2102 80.899) (end 109.2073 80.899) (width 0.25) (layer "F.Cu") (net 1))
 (segment (start 106.689 83.2202) (end 107.7878 83.2202) (width 0.25) (layer "F.Cu") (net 1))
 (segment (start 109.2073 82.7151) (end 109.2073 83.9927) (width 0.508) (layer "F.Cu") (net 1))
 (segment (start 113.0046 78.6003) (end 113.0046 77.7113) (width 0.508) (layer "F.Cu") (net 1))
 (segment (start 107.189 81.9202) (end 108.2102 80.899) (width 0.25) (layer "F.Cu") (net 1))
 (segment (start 99.7839 83.185) (end 99.7966 83.1723) (width 0.508) (layer "F.Cu") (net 1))
 (segment (start 111.911088 73.30231) (end 110.49 71.881222) (width 0.508) (layer "F.Cu") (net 1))
 (segment (start 111.911088 76.617788) (end 111.911088 73.30231) (width 0.508) (layer "F.Cu") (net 1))
 (segment (start 106.695307 87.380956) (end 106.695307 86.815271) (width 0.508) (layer "F.Cu") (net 1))
 (segment (start 109.364353 80.741947) (end 109.2073 80.899) (width 0.508) (layer "F.Cu") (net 1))
 (segment (start 104.639 82.5702) (end 103.3451 82.5702) (width 0.25) (layer "F.Cu") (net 1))
 (segment (start 113.0046 77.7113) (end 111.911088 76.617788) (width 0.508) (layer "F.Cu") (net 1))
 (segment (start 106.68 88.9) (end 106.695307 88.884693) (width 0.508) (layer "F.Cu") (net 1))
 (via (at 109.2073 83.9927) (size 0.8) (drill 0.4) (layers "F.Cu" "B.Cu") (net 1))
 (via (at 99.7839 84.0486) (size 0.8) (drill 0.4) (layers "F.Cu" "B.Cu") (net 1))
 (via (at 109.364353 79.925753) (size 0.8) (drill 0.4) (layers "F.Cu" "B.Cu") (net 1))
 (via (at 111.911088 73.30231) (size 0.8) (drill 0.4) (layers "F.Cu" "B.Cu") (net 1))
 (via (at 103.3272 82.5881) (size 0.8) (drill 0.4) (layers "F.Cu" "B.Cu") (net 1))
 (segment (start 109.1184 84.0486) (end 106.7435 84.0486) (width 0.508) (layer "B.Cu") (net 1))
 (segment (start 103.3399 84.0486) (end 100.349585 84.0486) (width 0.508) (layer "B.Cu") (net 1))
 (segment (start 100.349585 84.0486) (end 99.7839 84.0486) (width 0.508) (layer "B.Cu") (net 1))
 (segment (start 109.364353 75.849045) (end 111.911088 73.30231) (width 0.508) (layer "B.Cu") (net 1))
 (segment (start 106.7435 84.0486) (end 103.3399 84.0486) (width 0.508) (layer "B.Cu") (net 1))
 (segment (start 109.2962 79.8576) (end 109.364353 79.925753) (width 0.508) (layer "B.Cu") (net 1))
 (segment (start 106.7435 84.0486) (end 106.695307 84.096793) (width 0.508) (layer "B.Cu") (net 1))
 (segment (start 109.2962 79.8576) (end 109.2962 83.8708) (width 0.508) (layer "B.Cu") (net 1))
 (segment (start 103.3399 82.6008) (end 103.3399 84.0486) (width 0.508) (layer "B.Cu") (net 1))
 (segment (start 109.364353 79.925753) (end 109.364353 75.849045) (width 0.508) (layer "B.Cu") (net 1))
 (segment (start 109.2962 83.8708) (end 109.1184 84.0486) (width 0.508) (layer "B.Cu") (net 1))
 (segment (start 106.689 82.5702) (end 107.5107 82.5702) (width 0.25) (layer "F.Cu") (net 2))
 (segment (start 110.9853 84.4423) (end 109.22 86.2076) (width 0.508) (layer "F.Cu") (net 2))
 (segment (start 112.9919 80.899) (end 113.0046 80.8863) (width 0.508) (layer "F.Cu") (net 2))
 (segment (start 105.9994 82.5702) (end 105.3494 83.2202) (width 0.25) (layer "F.Cu") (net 2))
 (segment (start 111.8362 81.788) (end 111.270515 81.788) (width 0.508) (layer "F.Cu") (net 2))
 (segment (start 105.139 83.2202) (end 104.639 83.2202) (width 0.25) (layer "F.Cu") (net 2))
 (segment (start 108.2548 81.8261) (end 110.8543 81.8261) (width 0.25) (layer "F.Cu") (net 2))
 (segment (start 110.8543 81.8261) (end 110.9853 81.9571) (width 0.25) (layer "F.Cu") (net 2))
 (segment (start 110.9853 81.9571) (end 110.9853 82.7151) (width 0.25) (layer "F.Cu") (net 2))
 (segment (start 111.270515 81.788) (end 110.9853 81.788) (width 0.508) (layer "F.Cu") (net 2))
 (segment (start 106.689 82.5702) (end 105.9994 82.5702) (width 0.25) (layer "F.Cu") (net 2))
 (segment (start 110.49 75.818222) (end 110.49 78.0923) (width 0.508) (layer "F.Cu") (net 2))
 (segment (start 105.3494 83.2202) (end 105.139 83.2202) (width 0.25) (layer "F.Cu") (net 2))
 (segment (start 110.9853 80.899) (end 110.9853 82.7151) (width 0.508) (layer "F.Cu") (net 2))
 (segment (start 110.9853 80.899) (end 112.9919 80.899) (width 0.508) (layer "F.Cu") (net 2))
 (segment (start 107.5107 82.5702) (end 108.2548 81.8261) (width 0.25) (layer "F.Cu") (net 2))
 (segment (start 110.9853 81.788) (end 110.9853 81.9571) (width 0.25) (layer "F.Cu") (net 2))
 (segment (start 109.22 86.2076) (end 109.22 88.9) (width 0.508) (layer "F.Cu") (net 2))
 (segment (start 110.9853 80.899) (end 110.9853 81.657) (width 0.25) (layer "F.Cu") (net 2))
 (segment (start 110.9853 82.7151) (end 110.9853 84.4423) (width 0.508) (layer "F.Cu") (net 2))
 (segment (start 110.9853 81.657) (end 110.9853 81.788) (width 0.25) (layer "F.Cu") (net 2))
 (via (at 111.8362 81.788) (size 0.8) (drill 0.4) (layers "F.Cu" "B.Cu") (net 2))
 (via (at 110.49 78.0923) (size 0.8) (drill 0.4) (layers "F.Cu" "B.Cu") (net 2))
 (segment (start 110.49 78.0923) (end 110.49 80.4418) (width 0.508) (layer "B.Cu") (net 2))
 (segment (start 110.49 80.4418) (end 111.8362 81.788) (width 0.508) (layer "B.Cu") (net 2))
 (segment (start 104.2289 81.2702) (end 101.7241 81.2702) (width 0.25) (layer "F.Cu") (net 5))
 (segment (start 101.7241 81.2702) (end 100.6856 82.3087) (width 0.25) (layer "F.Cu") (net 5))
 (segment (start 104.1019 81.1432) (end 104.2289 81.2702) (width 0.25) (layer "F.Cu") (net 5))
 (segment (start 104.1019 80.2132) (end 104.1019 81.1432) (width 0.25) (layer "F.Cu") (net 5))
 (segment (start 105.41 71.7931) (end 104.1019 73.1012) (width 0.508) (layer "F.Cu") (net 5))
 (segment (start 105.41 69.468222) (end 105.41 71.7931) (width 0.508) (layer "F.Cu") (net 5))
 (segment (start 100.6856 82.3087) (end 100.6856 84.8955) (width 0.25) (layer "F.Cu") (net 5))
 (segment (start 104.1019 73.1012) (end 104.1019 80.2132) (width 0.508) (layer "F.Cu") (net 5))
 (segment (start 101.6 88.9) (end 101.6 85.0519) (width 0.508) (layer "F.Cu") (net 5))
 (segment (start 100.6856 84.8955) (end 100.8039 85.0138) (width 0.25) (layer "F.Cu") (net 5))
 (segment (start 100.8039 85.0138) (end 101.5619 85.0138) (width 0.25) (layer "F.Cu") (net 5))
 (segment (start 104.639 81.2702) (end 104.2289 81.2702) (width 0.25) (layer "F.Cu") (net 5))
 (segment (start 101.6 85.0519) (end 101.5619 85.0138) (width 0.508) (layer "F.Cu") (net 5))
 (segment (start 104.043798 81.824998) (end 102.163902 81.824998) (width 0.25) (layer "F.Cu") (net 6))
 (segment (start 104.139 81.9202) (end 104.043798 81.824998) (width 0.25) (layer "F.Cu") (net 6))
 (segment (start 102.3326 83.1723) (end 102.9843 83.824) (width 0.25) (layer "F.Cu") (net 6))
 (segment (start 104.14 86.233) (end 104.14 86.4743) (width 0.25) (layer "F.Cu") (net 6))
 (segment (start 105.139 81.9202) (end 104.639 81.9202) (width 0.25) (layer "F.Cu") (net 6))
 (segment (start 105.41 78.231222) (end 105.41 80.2386) (width 0.508) (layer "F.Cu") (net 6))
 (segment (start 105.41 80.2386) (end 105.41 81.6492) (width 0.25) (layer "F.Cu") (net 6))
 (segment (start 102.163902 81.824998) (end 101.5746 82.4143) (width 0.25) (layer "F.Cu") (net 6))
 (segment (start 105.41 75.818222) (end 105.41 78.231222) (width 0.508) (layer "F.Cu") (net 6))
 (segment (start 101.5746 83.1723) (end 102.3326 83.1723) (width 0.25) (layer "F.Cu") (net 6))
 (segment (start 104.639 81.9202) (end 104.139 81.9202) (width 0.25) (layer "F.Cu") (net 6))
 (segment (start 104.14 88.9) (end 104.14 86.4743) (width 0.508) (layer "F.Cu") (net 6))
 (segment (start 102.9843 85.0773) (end 104.14 86.233) (width 0.25) (layer "F.Cu") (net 6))
 (segment (start 105.41 81.6492) (end 105.139 81.9202) (width 0.25) (layer "F.Cu") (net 6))
 (segment (start 102.9843 83.824) (end 102.9843 85.0773) (width 0.25) (layer "F.Cu") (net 6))
 (segment (start 101.5746 82.4143) (end 101.5746 83.1723) (width 0.25) (layer "F.Cu") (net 6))
 (segment (start 109.2708 78.994) (end 111.4973 78.994) (width 0.25) (layer "F.Cu") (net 11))
 (segment (start 112.2466 79.7433) (end 113.0046 79.7433) (width 0.25) (layer "F.Cu") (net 11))
 (segment (start 106.9946 81.2702) (end 109.2708 78.994) (width 0.25) (layer "F.Cu") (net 11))
 (segment (start 106.689 81.2702) (end 106.9946 81.2702) (width 0.25) (layer "F.Cu") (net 11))
 (segment (start 111.4973 78.994) (end 112.2466 79.7433) (width 0.25) (layer "F.Cu") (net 11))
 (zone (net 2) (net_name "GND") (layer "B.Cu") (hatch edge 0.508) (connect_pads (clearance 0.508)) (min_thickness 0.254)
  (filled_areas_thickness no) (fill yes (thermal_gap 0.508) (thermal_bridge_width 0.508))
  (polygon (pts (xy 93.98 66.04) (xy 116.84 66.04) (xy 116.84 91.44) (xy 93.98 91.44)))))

